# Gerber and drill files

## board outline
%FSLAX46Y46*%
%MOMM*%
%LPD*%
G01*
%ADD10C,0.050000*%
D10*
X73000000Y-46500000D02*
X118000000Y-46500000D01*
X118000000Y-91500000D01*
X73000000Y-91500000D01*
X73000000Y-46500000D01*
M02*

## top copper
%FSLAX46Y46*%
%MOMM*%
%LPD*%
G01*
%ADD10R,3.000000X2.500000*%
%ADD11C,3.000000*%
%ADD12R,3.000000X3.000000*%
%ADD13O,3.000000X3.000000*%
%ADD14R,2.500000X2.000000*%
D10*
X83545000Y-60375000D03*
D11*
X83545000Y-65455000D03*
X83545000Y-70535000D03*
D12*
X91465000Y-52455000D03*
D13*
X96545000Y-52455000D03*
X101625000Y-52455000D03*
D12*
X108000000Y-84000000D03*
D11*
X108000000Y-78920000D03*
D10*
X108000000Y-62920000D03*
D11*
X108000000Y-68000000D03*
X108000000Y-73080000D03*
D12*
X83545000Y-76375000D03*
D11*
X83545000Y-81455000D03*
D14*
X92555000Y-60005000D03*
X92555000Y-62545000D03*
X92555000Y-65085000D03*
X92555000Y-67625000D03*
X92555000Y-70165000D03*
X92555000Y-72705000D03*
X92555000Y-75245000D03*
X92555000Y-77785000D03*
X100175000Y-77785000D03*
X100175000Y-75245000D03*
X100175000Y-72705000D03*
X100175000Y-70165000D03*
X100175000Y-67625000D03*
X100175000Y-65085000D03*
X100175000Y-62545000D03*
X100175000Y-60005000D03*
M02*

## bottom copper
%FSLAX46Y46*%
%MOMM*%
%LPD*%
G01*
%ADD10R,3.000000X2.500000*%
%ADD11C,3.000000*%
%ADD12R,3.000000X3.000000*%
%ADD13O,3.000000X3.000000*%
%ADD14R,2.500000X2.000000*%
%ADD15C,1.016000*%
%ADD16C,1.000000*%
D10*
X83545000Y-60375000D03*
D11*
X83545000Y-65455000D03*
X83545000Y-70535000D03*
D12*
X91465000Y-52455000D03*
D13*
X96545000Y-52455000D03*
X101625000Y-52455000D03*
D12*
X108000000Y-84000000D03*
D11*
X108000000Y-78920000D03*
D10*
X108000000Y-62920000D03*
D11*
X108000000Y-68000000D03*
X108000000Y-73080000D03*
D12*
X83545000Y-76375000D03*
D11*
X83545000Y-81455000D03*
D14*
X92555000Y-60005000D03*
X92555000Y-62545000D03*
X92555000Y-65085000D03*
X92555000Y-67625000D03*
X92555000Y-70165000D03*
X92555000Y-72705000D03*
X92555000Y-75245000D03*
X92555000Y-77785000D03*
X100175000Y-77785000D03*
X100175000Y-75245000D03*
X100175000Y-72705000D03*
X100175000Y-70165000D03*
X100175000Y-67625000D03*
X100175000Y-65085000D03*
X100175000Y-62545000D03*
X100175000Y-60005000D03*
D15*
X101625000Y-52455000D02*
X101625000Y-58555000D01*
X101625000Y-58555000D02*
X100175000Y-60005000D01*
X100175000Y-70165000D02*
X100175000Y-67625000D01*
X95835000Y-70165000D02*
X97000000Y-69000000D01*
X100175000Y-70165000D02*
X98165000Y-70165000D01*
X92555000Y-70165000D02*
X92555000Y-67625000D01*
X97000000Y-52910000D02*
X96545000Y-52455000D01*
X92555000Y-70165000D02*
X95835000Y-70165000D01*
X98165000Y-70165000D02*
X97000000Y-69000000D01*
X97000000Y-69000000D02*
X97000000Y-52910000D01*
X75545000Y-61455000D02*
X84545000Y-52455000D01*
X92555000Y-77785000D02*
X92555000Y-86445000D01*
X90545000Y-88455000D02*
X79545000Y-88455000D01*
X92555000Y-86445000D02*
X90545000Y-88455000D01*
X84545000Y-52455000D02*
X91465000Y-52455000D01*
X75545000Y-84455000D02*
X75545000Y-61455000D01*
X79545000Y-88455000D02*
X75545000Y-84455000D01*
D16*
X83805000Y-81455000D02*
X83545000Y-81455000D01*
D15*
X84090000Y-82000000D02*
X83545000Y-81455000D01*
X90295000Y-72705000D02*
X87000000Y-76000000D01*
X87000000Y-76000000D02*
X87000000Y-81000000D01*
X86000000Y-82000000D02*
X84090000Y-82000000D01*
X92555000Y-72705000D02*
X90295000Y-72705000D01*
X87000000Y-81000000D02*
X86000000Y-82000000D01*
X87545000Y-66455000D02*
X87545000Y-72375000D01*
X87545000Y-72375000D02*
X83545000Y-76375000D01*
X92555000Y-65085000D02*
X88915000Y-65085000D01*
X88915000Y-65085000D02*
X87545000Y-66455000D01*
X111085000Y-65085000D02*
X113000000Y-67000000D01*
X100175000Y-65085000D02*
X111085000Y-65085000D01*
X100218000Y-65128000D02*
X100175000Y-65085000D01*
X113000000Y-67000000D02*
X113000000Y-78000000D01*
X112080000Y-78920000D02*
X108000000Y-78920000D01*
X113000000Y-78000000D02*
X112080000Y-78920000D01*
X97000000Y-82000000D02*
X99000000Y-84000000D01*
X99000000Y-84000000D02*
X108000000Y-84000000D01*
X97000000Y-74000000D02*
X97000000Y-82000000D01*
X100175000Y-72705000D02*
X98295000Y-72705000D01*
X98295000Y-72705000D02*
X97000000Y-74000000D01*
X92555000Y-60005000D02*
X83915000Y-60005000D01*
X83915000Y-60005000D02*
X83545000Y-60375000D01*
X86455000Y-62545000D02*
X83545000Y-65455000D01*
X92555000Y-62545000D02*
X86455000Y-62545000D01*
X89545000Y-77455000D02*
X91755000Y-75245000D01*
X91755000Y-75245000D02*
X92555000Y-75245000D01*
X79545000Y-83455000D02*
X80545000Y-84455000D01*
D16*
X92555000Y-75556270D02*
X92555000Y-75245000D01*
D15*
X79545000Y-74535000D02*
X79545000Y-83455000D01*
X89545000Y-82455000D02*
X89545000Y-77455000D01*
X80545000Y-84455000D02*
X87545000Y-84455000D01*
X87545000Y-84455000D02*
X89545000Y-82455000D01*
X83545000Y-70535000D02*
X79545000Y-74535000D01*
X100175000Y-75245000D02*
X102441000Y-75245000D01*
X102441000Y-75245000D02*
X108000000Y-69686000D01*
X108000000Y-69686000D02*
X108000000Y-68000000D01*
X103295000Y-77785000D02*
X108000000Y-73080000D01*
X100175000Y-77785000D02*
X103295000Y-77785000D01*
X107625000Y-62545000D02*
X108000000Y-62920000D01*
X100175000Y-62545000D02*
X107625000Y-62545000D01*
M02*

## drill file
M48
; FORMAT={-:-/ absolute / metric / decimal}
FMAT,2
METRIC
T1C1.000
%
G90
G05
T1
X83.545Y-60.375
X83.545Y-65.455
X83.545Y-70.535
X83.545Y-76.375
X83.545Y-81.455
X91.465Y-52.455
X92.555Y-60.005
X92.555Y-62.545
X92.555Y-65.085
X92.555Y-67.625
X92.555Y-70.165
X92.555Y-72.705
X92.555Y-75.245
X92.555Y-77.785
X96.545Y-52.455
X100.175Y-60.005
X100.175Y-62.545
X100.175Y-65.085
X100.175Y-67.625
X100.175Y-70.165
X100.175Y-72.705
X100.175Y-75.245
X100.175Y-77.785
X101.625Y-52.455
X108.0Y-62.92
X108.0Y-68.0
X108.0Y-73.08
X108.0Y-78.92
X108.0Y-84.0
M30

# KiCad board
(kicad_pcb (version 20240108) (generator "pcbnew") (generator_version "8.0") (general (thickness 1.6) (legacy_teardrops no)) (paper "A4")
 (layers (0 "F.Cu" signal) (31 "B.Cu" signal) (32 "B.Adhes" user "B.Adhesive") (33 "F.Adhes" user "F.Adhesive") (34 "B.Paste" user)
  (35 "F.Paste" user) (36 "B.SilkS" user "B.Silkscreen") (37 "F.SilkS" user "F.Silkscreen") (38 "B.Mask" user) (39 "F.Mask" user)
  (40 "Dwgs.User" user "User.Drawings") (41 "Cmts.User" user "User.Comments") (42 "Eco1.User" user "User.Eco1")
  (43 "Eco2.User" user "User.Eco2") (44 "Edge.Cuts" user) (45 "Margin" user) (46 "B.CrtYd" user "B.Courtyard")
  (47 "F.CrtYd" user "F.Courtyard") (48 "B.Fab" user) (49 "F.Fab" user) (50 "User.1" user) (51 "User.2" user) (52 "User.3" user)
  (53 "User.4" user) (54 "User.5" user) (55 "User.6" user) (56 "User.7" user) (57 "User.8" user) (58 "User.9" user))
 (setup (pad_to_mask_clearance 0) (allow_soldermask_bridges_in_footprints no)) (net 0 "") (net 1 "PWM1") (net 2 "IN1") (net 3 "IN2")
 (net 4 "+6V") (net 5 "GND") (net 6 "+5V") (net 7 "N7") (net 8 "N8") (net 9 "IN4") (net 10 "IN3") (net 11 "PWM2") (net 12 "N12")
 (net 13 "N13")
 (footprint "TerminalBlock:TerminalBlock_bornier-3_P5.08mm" (layer "F.Cu") (at 83.545 60.375 -90)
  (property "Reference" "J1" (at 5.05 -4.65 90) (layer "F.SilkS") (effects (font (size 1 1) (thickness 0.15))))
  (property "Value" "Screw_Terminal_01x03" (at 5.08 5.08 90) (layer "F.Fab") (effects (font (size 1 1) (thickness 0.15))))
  (pad "1" thru_hole rect (at 0 0 270) (size 2.5 3) (drill 1) (layers "*.Cu" "*.Mask") (remove_unused_layers no) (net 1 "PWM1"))
  (pad "2" thru_hole circle (at 5.08 0 270) (size 3 3) (drill 1) (layers "*.Cu" "*.Mask") (remove_unused_layers no) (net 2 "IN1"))
  (pad "3" thru_hole circle (at 10.16 0 270) (size 3 3) (drill 1) (layers "*.Cu" "*.Mask") (remove_unused_layers no) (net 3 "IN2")))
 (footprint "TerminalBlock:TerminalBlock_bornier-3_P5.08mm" (layer "F.Cu") (at 91.465 52.455)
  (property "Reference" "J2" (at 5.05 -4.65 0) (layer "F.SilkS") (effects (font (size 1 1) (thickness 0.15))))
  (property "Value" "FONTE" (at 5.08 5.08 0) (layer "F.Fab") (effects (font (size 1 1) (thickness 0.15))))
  (pad "1" thru_hole rect (at 0 0) (size 3 3) (drill 1) (layers "*.Cu" "*.Mask") (remove_unused_layers no) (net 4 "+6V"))
  (pad "2" thru_hole oval (at 5.08 0) (size 3 3) (drill 1) (layers "*.Cu" "*.Mask" "Eco2.User") (remove_unused_layers no) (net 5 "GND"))
  (pad "3" thru_hole oval (at 10.16 0) (size 3 3) (drill 1) (layers "*.Cu" "*.Mask") (remove_unused_layers no) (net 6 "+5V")))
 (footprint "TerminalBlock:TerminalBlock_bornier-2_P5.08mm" (layer "F.Cu") (at 108 84 90)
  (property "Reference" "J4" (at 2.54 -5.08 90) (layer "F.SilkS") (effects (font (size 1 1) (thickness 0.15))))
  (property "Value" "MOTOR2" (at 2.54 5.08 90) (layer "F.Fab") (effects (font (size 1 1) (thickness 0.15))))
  (pad "1" thru_hole rect (at 0 0 90) (size 3 3) (drill 1) (layers "*.Cu" "*.Mask") (remove_unused_layers no) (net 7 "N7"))
  (pad "2" thru_hole circle (at 5.08 0 90) (size 3 3) (drill 1) (layers "*.Cu" "*.Mask") (remove_unused_layers no) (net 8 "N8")))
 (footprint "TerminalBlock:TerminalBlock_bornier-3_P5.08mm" (layer "F.Cu") (at 108 62.92 -90)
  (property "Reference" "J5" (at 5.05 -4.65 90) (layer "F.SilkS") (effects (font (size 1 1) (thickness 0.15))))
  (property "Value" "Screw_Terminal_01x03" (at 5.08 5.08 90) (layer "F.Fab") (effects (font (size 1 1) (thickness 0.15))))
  (pad "1" thru_hole rect (at 0 0 270) (size 2.5 3) (drill 1) (layers "*.Cu" "*.Mask") (remove_unused_layers no) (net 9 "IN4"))
  (pad "2" thru_hole circle (at 5.08 0 270) (size 3 3) (drill 1) (layers "*.Cu" "*.Mask" "Eco1.User") (remove_unused_layers no)
   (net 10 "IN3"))
  (pad "3" thru_hole circle (at 10.16 0 270) (size 3 3) (drill 1) (layers "*.Cu" "*.Mask") (remove_unused_layers no) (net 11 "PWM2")))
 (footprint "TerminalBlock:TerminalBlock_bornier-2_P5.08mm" (layer "F.Cu") (at 83.545 76.375 -90)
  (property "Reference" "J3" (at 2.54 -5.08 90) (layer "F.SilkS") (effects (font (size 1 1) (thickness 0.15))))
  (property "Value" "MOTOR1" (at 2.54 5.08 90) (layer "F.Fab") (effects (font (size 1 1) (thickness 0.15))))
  (pad "1" thru_hole rect (at 0 0 270) (size 3 3) (drill 1) (layers "*.Cu" "*.Mask") (remove_unused_layers no) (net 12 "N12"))
  (pad "2" thru_hole circle (at 5.08 0 270) (size 3 3) (drill 1) (layers "*.Cu" "*.Mask") (remove_unused_layers no) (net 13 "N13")))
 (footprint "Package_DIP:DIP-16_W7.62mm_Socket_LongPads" (layer "F.Cu") (at 92.555 60.005)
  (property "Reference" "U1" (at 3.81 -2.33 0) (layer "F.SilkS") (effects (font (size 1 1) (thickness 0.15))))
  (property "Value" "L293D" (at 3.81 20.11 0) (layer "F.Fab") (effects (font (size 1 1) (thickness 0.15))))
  (pad "1" thru_hole rect (at 0 0) (size 2.5 2) (drill 1) (layers "*.Cu" "B.Mask") (remove_unused_layers no) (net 1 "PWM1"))
  (pad "2" thru_hole rect (at 0 2.54) (size 2.5 2) (drill 1) (layers "*.Cu" "*.Mask") (remove_unused_layers no) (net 2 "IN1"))
  (pad "3" thru_hole rect (at 0 5.08) (size 2.5 2) (drill 1) (layers "*.Cu" "*.Mask") (remove_unused_layers no) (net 12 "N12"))
  (pad "4" thru_hole rect (at 0 7.62) (size 2.5 2) (drill 1) (layers "*.Cu" "*.Mask") (remove_unused_layers no) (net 5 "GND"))
  (pad "5" thru_hole rect (at 0 10.16) (size 2.5 2) (drill 1) (layers "*.Cu" "*.Mask") (remove_unused_layers no) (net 5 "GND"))
  (pad "6" thru_hole rect (at 0 12.7) (size 2.5 2) (drill 1) (layers "*.Cu" "*.Mask") (remove_unused_layers no) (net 13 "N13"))
  (pad "7" thru_hole rect (at 0 15.24) (size 2.5 2) (drill 1) (layers "*.Cu" "*.Mask") (remove_unused_layers no) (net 3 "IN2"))
  (pad "8" thru_hole rect (at 0 17.78) (size 2.5 2) (drill 1) (layers "*.Cu" "*.Mask") (remove_unused_layers no) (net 4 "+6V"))
  (pad "9" thru_hole rect (at 7.62 17.78) (size 2.5 2) (drill 1) (layers "*.Cu" "*.Mask") (remove_unused_layers no) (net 11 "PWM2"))
  (pad "10" thru_hole rect (at 7.62 15.24) (size 2.5 2) (drill 1) (layers "*.Cu" "*.Mask") (remove_unused_layers no) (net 10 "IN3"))
  (pad "11" thru_hole rect (at 7.62 12.7) (size 2.5 2) (drill 1) (layers "*.Cu" "*.Mask") (remove_unused_layers no) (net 7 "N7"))
  (pad "12" thru_hole rect (at 7.62 10.16) (size 2.5 2) (drill 1) (layers "*.Cu" "*.Mask") (remove_unused_layers no) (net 5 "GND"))
  (pad "13" thru_hole rect (at 7.62 7.62) (size 2.5 2) (drill 1) (layers "*.Cu" "*.Mask") (remove_unused_layers no) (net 5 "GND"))
  (pad "14" thru_hole rect (at 7.62 5.08) (size 2.5 2) (drill 1) (layers "*.Cu" "*.Mask") (remove_unused_layers no) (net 8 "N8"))
  (pad "15" thru_hole rect (at 7.62 2.54) (size 2.5 2) (drill 1) (layers "*.Cu" "*.Mask") (remove_unused_layers no) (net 9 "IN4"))
  (pad "16" thru_hole rect (at 7.62 0) (size 2.5 2) (drill 1) (layers "*.Cu" "*.Mask") (remove_unused_layers no) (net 6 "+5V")))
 (gr_rect (start 73 46.5) (end 118 91.5) (stroke (width 0.05) (type default)) (fill none) (layer "Edge.Cuts"))
 (segment (start 101.625 52.455) (end 101.625 58.555) (width 1.016) (layer "B.Cu") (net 6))
 (segment (start 101.625 58.555) (end 100.175 60.005) (width 1.016) (layer "B.Cu") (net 6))
 (segment (start 100.175 70.165) (end 100.175 67.625) (width 1.016) (layer "B.Cu") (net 5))
 (segment (start 95.835 70.165) (end 97 69) (width 1.016) (layer "B.Cu") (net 5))
 (segment (start 100.175 70.165) (end 98.165 70.165) (width 1.016) (layer "B.Cu") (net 5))
 (segment (start 92.555 70.165) (end 92.555 67.625) (width 1.016) (layer "B.Cu") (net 5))
 (segment (start 97 52.91) (end 96.545 52.455) (width 1.016) (layer "B.Cu") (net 5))
 (segment (start 92.555 70.165) (end 95.835 70.165) (width 1.016) (layer "B.Cu") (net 5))
 (segment (start 98.165 70.165) (end 97 69) (width 1.016) (layer "B.Cu") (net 5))
 (segment (start 97 69) (end 97 52.91) (width 1.016) (layer "B.Cu") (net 5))
 (segment (start 75.545 61.455) (end 84.545 52.455) (width 1.016) (layer "B.Cu") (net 4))
 (segment (start 92.555 77.785) (end 92.555 86.445) (width 1.016) (layer "B.Cu") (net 4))
 (segment (start 90.545 88.455) (end 79.545 88.455) (width 1.016) (layer "B.Cu") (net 4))
 (segment (start 92.555 86.445) (end 90.545 88.455) (width 1.016) (layer "B.Cu") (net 4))
 (segment (start 84.545 52.455) (end 91.465 52.455) (width 1.016) (layer "B.Cu") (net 4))
 (segment (start 75.545 84.455) (end 75.545 61.455) (width 1.016) (layer "B.Cu") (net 4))
 (segment (start 79.545 88.455) (end 75.545 84.455) (width 1.016) (layer "B.Cu") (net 4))
 (segment (start 83.805 81.455) (end 83.545 81.455) (width 1) (layer "B.Cu") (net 13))
 (segment (start 84.09 82) (end 83.545 81.455) (width 1.016) (layer "B.Cu") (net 13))
 (segment (start 90.295 72.705) (end 87 76) (width 1.016) (layer "B.Cu") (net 13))
 (segment (start 87 76) (end 87 81) (width 1.016) (layer "B.Cu") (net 13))
 (segment (start 86 82) (end 84.09 82) (width 1.016) (layer "B.Cu") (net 13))
 (segment (start 92.555 72.705) (end 90.295 72.705) (width 1.016) (layer "B.Cu") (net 13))
 (segment (start 87 81) (end 86 82) (width 1.016) (layer "B.Cu") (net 13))
 (segment (start 87.545 66.455) (end 87.545 72.375) (width 1.016) (layer "B.Cu") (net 12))
 (segment (start 87.545 72.375) (end 83.545 76.375) (width 1.016) (layer "B.Cu") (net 12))
 (segment (start 92.555 65.085) (end 88.915 65.085) (width 1.016) (layer "B.Cu") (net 12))
 (segment (start 88.915 65.085) (end 87.545 66.455) (width 1.016) (layer "B.Cu") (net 12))
 (segment (start 111.085 65.085) (end 113 67) (width 1.016) (layer "B.Cu") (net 8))
 (segment (start 100.175 65.085) (end 111.085 65.085) (width 1.016) (layer "B.Cu") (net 8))
 (segment (start 100.218 65.128) (end 100.175 65.085) (width 1.016) (layer "B.Cu") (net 8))
 (segment (start 113 67) (end 113 78) (width 1.016) (layer "B.Cu") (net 8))
 (segment (start 112.08 78.92) (end 108 78.92) (width 1.016) (layer "B.Cu") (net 8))
 (segment (start 113 78) (end 112.08 78.92) (width 1.016) (layer "B.Cu") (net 8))
 (segment (start 97 82) (end 99 84) (width 1.016) (layer "B.Cu") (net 7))
 (segment (start 99 84) (end 108 84) (width 1.016) (layer "B.Cu") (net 7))
 (segment (start 97 74) (end 97 82) (width 1.016) (layer "B.Cu") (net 7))
 (segment (start 100.175 72.705) (end 98.295 72.705) (width 1.016) (layer "B.Cu") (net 7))
 (segment (start 98.295 72.705) (end 97 74) (width 1.016) (layer "B.Cu") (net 7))
 (segment (start 92.555 60.005) (end 83.915 60.005) (width 1.016) (layer "B.Cu") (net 1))
 (segment (start 83.915 60.005) (end 83.545 60.375) (width 1.016) (layer "B.Cu") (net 1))
 (segment (start 86.455 62.545) (end 83.545 65.455) (width 1.016) (layer "B.Cu") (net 2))
 (segment (start 92.555 62.545) (end 86.455 62.545) (width 1.016) (layer "B.Cu") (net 2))
 (segment (start 89.545 77.455) (end 91.755 75.245) (width 1.016) (layer "B.Cu") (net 3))
 (segment (start 91.755 75.245) (end 92.555 75.245) (width 1.016) (layer "B.Cu") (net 3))
 (segment (start 79.545 83.455) (end 80.545 84.455) (width 1.016) (layer "B.Cu") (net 3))
 (segment (start 92.555 75.55627) (end 92.555 75.245) (width 1) (layer "B.Cu") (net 3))
 (segment (start 79.545 74.535) (end 79.545 83.455) (width 1.016) (layer "B.Cu") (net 3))
 (segment (start 89.545 82.455) (end 89.545 77.455) (width 1.016) (layer "B.Cu") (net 3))
 (segment (start 80.545 84.455) (end 87.545 84.455) (width 1.016) (layer "B.Cu") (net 3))
 (segment (start 87.545 84.455) (end 89.545 82.455) (width 1.016) (layer "B.Cu") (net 3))
 (segment (start 83.545 70.535) (end 79.545 74.535) (width 1.016) (layer "B.Cu") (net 3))
 (segment (start 100.175 75.245) (end 102.441 75.245) (width 1.016) (layer "B.Cu") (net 10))
 (segment (start 102.441 75.245) (end 108 69.686) (width 1.016) (layer "B.Cu") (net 10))
 (segment (start 108 69.686) (end 108 68) (width 1.016) (layer "B.Cu") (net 10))
 (segment (start 103.295 77.785) (end 108 73.08) (width 1.016) (layer "B.Cu") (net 11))
 (segment (start 100.175 77.785) (end 103.295 77.785) (width 1.016) (layer "B.Cu") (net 11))
 (segment (start 107.625 62.545) (end 108 62.92) (width 1.016) (layer "B.Cu") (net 9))
 (segment (start 100.175 62.545) (end 107.625 62.545) (width 1.016) (layer "B.Cu") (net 9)))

